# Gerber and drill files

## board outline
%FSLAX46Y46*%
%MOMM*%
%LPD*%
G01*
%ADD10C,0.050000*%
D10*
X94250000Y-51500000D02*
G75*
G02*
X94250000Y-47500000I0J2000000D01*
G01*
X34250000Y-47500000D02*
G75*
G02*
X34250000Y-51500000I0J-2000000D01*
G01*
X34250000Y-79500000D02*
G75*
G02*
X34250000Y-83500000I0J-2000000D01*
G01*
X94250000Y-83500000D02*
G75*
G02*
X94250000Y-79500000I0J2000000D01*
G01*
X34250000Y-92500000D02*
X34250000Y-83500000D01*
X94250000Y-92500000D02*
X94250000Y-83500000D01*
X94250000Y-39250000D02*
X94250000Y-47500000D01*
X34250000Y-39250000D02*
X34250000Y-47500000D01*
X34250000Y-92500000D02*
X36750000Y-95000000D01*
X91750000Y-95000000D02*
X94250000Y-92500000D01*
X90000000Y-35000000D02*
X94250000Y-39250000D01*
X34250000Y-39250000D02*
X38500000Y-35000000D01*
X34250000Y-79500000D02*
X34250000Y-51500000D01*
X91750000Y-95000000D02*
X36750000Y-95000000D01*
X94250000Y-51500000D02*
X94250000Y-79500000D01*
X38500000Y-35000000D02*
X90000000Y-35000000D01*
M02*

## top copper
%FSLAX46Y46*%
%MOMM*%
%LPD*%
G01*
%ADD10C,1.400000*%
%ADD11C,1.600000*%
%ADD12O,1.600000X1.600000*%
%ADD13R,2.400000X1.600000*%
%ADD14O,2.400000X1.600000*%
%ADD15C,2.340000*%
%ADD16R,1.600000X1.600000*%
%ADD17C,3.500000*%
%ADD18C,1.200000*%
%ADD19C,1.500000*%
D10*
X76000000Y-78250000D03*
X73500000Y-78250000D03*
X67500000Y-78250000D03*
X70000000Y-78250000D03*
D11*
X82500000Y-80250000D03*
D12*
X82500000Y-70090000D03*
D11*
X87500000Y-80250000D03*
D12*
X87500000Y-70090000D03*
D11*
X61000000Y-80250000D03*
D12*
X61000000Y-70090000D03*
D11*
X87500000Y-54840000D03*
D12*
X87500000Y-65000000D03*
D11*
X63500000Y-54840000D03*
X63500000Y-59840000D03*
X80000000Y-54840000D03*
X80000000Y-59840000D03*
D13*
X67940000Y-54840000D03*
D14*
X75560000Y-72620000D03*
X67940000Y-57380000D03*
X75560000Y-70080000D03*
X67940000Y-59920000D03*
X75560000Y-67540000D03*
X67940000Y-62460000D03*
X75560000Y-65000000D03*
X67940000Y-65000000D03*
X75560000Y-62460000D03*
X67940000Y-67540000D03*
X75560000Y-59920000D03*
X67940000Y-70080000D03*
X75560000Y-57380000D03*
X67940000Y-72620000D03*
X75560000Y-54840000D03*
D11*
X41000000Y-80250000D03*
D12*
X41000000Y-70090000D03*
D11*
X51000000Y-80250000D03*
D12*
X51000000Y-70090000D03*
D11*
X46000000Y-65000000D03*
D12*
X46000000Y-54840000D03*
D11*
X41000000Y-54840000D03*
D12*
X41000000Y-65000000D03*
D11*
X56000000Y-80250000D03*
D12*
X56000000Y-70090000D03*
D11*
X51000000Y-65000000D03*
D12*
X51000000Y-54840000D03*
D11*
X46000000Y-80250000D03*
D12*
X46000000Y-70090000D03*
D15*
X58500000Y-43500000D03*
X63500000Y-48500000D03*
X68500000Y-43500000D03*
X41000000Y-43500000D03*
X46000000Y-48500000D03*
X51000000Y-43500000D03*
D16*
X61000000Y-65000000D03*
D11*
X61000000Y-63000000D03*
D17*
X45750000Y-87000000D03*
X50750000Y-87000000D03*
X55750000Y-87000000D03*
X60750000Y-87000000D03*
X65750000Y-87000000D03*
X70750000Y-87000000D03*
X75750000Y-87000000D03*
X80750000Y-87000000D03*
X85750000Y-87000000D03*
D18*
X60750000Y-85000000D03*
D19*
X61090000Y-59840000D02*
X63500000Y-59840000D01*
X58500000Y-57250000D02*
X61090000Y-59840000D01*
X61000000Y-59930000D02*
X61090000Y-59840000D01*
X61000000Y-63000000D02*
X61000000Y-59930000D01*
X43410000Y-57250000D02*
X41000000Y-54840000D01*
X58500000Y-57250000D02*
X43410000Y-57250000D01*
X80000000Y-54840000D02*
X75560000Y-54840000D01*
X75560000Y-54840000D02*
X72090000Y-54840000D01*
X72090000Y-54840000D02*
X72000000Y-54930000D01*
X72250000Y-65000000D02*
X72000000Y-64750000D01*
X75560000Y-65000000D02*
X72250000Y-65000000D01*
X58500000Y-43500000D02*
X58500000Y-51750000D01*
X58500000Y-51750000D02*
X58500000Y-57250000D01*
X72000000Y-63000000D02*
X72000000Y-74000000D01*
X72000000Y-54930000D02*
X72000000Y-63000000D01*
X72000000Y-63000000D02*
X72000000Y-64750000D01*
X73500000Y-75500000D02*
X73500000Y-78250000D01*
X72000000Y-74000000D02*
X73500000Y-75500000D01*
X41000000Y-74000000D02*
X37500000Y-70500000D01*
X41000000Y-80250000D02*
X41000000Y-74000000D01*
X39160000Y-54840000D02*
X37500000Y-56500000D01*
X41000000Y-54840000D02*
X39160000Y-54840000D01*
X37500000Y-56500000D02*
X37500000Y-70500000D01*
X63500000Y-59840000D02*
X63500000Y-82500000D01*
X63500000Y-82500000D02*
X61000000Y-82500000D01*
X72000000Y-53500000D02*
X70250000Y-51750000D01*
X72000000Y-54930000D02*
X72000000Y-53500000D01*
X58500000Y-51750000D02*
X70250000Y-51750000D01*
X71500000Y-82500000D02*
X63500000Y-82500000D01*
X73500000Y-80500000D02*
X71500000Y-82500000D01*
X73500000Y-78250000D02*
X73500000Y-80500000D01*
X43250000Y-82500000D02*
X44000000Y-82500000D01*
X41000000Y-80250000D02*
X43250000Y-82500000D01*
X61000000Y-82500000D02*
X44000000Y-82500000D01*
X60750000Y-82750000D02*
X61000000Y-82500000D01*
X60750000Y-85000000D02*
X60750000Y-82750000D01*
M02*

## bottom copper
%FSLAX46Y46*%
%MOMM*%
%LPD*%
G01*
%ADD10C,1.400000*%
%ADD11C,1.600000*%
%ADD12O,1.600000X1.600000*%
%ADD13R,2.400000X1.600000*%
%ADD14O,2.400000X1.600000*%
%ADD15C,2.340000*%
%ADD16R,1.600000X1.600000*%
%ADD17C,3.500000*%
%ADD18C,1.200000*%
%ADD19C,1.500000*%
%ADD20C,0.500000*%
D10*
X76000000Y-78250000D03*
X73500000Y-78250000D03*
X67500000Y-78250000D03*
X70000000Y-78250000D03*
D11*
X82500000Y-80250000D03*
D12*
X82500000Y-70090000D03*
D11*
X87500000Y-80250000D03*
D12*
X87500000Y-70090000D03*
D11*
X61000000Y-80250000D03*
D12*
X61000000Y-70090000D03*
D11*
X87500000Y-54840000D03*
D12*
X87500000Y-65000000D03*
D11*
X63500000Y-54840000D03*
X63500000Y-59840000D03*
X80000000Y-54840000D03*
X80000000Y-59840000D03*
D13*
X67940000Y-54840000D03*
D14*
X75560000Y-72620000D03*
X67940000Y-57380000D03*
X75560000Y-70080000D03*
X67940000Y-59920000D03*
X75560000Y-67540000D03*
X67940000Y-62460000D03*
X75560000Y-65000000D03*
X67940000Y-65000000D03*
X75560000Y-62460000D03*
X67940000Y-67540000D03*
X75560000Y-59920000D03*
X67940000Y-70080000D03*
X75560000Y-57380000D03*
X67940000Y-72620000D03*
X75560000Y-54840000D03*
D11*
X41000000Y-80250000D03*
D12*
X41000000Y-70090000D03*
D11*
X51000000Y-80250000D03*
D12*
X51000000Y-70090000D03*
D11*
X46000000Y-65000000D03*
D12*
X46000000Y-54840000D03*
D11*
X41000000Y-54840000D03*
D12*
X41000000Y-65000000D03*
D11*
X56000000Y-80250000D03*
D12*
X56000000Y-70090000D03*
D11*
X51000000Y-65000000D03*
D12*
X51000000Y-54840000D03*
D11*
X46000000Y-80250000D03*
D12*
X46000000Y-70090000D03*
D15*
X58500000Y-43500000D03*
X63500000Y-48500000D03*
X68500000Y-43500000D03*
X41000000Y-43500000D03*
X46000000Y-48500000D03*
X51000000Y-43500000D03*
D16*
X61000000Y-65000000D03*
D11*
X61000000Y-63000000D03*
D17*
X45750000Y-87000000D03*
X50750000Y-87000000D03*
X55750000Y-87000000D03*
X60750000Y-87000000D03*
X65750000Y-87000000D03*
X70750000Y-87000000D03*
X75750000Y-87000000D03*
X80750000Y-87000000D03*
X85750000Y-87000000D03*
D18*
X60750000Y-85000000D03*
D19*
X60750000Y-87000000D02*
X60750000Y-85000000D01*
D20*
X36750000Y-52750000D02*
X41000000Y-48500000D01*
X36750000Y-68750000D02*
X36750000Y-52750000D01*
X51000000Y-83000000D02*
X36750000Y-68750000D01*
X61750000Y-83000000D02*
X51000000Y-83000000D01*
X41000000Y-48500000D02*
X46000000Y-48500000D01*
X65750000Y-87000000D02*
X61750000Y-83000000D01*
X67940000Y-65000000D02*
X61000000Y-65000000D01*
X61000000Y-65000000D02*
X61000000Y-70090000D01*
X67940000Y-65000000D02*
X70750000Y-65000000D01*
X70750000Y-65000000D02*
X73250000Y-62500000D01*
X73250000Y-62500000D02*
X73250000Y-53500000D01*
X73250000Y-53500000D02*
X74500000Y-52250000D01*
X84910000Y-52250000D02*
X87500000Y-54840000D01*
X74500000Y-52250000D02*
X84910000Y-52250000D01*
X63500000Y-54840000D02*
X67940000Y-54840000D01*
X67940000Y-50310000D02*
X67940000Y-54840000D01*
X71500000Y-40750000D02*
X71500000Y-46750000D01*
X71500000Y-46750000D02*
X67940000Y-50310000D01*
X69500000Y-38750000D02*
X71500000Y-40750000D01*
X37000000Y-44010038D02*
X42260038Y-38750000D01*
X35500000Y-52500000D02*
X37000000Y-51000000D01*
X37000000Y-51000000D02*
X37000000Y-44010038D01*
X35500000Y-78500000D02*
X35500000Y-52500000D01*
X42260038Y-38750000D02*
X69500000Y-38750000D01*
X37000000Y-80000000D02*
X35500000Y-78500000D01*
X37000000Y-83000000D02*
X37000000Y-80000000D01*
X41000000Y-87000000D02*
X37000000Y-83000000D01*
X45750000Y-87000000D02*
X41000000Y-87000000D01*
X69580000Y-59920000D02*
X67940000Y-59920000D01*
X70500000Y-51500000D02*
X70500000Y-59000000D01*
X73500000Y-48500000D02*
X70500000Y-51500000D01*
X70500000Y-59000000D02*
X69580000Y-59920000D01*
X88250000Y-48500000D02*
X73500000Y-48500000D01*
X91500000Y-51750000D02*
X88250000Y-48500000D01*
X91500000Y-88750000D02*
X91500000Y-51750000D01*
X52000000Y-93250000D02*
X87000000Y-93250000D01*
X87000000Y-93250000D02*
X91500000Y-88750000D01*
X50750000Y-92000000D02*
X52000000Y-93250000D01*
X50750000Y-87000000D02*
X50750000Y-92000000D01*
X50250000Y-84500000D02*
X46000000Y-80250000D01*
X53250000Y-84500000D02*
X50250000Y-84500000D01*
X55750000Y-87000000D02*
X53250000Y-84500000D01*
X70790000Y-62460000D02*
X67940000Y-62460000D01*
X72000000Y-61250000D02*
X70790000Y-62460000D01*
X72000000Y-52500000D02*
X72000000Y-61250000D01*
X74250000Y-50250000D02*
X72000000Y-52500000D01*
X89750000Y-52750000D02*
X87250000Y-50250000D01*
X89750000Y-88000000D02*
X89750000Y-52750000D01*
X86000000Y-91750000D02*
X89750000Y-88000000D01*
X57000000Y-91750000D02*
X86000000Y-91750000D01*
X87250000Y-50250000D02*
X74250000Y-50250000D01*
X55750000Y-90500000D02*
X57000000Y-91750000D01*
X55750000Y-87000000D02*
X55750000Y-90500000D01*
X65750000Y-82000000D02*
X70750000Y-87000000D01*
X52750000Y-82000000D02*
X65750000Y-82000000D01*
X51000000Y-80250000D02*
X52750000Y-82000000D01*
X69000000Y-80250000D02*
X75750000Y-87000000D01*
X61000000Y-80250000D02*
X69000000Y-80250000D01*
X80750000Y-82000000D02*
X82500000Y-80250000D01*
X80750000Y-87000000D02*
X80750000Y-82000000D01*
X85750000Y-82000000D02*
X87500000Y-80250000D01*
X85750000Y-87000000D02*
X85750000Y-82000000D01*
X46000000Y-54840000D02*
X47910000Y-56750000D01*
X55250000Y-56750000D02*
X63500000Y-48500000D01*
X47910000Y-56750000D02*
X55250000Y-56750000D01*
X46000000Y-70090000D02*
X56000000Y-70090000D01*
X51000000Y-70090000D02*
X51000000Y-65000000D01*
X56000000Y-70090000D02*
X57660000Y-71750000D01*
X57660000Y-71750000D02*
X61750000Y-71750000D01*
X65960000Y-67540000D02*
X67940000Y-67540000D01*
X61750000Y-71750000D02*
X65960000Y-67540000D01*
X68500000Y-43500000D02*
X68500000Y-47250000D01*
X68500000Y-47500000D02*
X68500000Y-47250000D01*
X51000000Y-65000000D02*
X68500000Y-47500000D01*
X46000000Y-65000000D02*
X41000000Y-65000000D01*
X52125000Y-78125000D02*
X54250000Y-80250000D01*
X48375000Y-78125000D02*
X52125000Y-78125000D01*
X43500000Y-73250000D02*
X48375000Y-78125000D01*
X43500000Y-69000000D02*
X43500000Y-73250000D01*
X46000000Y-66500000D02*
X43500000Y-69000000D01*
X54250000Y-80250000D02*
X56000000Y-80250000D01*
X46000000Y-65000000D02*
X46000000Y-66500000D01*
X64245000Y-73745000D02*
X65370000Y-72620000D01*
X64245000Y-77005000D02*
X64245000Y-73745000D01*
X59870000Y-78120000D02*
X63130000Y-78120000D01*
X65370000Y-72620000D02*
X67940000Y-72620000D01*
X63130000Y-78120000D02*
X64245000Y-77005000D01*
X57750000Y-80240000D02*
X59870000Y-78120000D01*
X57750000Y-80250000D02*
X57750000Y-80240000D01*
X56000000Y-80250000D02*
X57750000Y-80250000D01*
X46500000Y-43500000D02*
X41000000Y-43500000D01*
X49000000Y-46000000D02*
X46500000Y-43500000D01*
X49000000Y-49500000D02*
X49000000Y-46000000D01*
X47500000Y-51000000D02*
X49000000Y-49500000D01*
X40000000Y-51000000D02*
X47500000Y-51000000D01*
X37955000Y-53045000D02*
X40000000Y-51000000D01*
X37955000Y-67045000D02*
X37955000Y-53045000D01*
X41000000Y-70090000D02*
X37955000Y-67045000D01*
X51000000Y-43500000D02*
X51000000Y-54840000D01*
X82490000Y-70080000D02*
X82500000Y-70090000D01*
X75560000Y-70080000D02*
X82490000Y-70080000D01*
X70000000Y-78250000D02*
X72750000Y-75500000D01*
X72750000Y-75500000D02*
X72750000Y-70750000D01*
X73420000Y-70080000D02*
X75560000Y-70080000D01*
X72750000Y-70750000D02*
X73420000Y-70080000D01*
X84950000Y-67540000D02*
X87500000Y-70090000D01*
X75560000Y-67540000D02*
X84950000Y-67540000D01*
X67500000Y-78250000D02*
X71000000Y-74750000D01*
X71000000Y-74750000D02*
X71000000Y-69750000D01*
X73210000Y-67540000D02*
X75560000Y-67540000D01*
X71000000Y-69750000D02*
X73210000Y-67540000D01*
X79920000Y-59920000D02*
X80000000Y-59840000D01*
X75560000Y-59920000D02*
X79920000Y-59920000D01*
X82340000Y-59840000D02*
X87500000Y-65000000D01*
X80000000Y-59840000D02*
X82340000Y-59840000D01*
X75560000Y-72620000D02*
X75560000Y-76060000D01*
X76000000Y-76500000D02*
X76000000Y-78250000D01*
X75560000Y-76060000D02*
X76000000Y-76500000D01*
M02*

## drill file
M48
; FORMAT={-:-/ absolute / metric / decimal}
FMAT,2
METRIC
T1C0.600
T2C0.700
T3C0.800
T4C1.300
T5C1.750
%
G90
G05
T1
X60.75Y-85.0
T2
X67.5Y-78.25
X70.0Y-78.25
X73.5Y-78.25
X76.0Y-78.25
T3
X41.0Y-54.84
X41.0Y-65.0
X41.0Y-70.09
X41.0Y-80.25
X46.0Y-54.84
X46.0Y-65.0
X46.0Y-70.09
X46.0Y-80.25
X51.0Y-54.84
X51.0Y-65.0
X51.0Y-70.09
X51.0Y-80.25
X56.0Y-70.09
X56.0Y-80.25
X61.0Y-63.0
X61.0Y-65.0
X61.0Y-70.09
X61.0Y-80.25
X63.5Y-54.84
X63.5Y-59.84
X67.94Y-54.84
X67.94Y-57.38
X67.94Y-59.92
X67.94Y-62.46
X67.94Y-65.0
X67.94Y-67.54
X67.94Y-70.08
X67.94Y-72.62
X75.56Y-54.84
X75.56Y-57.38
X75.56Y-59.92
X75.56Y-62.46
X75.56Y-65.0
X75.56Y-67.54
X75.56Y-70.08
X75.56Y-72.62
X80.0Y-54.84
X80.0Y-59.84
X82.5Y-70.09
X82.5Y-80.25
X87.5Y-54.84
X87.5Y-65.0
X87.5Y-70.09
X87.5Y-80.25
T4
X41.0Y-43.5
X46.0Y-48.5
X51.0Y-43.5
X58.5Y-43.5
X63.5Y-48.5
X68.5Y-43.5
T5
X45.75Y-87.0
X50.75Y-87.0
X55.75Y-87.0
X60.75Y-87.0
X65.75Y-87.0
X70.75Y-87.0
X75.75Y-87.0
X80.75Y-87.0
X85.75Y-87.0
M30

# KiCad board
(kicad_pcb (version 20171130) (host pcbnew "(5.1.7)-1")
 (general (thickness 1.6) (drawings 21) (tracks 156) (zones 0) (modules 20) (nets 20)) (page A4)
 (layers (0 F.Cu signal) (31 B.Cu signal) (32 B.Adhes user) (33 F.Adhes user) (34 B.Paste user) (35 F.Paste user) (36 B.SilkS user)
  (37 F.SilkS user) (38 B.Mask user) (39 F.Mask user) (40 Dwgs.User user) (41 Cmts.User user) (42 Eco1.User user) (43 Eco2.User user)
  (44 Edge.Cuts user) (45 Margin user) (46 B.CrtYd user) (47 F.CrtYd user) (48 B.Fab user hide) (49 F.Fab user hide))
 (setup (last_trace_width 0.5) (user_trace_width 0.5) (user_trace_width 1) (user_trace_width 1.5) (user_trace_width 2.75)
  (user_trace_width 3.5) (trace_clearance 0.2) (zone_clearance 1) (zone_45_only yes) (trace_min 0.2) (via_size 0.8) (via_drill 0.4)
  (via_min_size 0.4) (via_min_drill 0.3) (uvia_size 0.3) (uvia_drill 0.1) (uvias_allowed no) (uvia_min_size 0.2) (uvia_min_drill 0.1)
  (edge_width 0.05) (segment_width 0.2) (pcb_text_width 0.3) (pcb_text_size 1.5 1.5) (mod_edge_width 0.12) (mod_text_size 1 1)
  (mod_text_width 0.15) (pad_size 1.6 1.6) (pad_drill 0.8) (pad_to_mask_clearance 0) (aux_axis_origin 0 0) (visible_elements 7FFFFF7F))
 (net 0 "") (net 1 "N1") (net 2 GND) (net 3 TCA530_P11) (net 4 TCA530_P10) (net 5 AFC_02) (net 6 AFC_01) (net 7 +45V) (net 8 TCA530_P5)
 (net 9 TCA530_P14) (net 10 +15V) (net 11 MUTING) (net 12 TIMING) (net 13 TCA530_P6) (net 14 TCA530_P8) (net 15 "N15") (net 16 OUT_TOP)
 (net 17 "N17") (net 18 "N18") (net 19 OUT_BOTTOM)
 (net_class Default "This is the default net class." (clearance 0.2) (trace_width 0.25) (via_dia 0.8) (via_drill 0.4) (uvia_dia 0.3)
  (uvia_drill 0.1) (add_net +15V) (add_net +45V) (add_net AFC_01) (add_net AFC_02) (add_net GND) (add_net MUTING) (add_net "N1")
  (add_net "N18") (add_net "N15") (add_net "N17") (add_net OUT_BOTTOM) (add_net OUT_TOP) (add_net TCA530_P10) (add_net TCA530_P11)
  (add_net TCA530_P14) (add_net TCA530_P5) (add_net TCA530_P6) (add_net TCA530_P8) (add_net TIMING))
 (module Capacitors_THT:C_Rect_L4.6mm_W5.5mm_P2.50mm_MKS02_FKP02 (layer F.Cu) (at 76 78.25 180)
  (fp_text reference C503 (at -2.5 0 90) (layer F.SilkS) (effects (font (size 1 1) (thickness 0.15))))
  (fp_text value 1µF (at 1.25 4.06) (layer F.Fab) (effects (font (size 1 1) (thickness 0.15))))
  (pad 1 thru_hole circle (at 0 0 180) (size 1.4 1.4) (drill 0.7) (layers *.Cu *.Mask) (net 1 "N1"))
  (pad 2 thru_hole circle (at 2.5 0 180) (size 1.4 1.4) (drill 0.7) (layers *.Cu *.Mask) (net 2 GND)))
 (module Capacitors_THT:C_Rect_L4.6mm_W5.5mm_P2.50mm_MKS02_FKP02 (layer F.Cu) (at 67.5 78.25)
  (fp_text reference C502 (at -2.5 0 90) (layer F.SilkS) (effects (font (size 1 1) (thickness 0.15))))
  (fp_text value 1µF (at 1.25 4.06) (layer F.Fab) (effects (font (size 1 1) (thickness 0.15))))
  (pad 1 thru_hole circle (at 0 0) (size 1.4 1.4) (drill 0.7) (layers *.Cu *.Mask) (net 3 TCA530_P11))
  (pad 2 thru_hole circle (at 2.5 0) (size 1.4 1.4) (drill 0.7) (layers *.Cu *.Mask) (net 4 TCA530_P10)))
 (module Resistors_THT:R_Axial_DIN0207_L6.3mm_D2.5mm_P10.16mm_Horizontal (layer F.Cu) (at 82.5 80.25 90)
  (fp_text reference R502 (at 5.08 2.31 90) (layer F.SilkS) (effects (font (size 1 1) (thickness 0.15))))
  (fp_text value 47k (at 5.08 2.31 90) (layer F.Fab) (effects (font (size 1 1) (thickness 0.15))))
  (pad 1 thru_hole circle (at 0 0 90) (size 1.6 1.6) (drill 0.8) (layers *.Cu *.Mask) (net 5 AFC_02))
  (pad 2 thru_hole oval (at 10.16 0 90) (size 1.6 1.6) (drill 0.8) (layers *.Cu *.Mask) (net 4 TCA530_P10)))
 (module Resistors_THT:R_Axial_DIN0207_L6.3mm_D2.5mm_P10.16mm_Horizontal (layer F.Cu) (at 87.5 80.25 90)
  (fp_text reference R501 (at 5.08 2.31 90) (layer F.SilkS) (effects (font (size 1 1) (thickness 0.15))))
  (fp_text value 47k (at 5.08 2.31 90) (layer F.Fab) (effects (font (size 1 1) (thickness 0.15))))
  (pad 1 thru_hole circle (at 0 0 90) (size 1.6 1.6) (drill 0.8) (layers *.Cu *.Mask) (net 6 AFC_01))
  (pad 2 thru_hole oval (at 10.16 0 90) (size 1.6 1.6) (drill 0.8) (layers *.Cu *.Mask) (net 3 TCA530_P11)))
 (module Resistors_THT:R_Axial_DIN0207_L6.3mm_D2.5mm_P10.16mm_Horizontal (layer F.Cu) (at 61 80.25 90)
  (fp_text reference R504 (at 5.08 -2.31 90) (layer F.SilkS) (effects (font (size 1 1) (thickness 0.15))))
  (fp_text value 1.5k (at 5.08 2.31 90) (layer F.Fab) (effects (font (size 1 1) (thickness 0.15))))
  (pad 1 thru_hole circle (at 0 0 90) (size 1.6 1.6) (drill 0.8) (layers *.Cu *.Mask) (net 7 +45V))
  (pad 2 thru_hole oval (at 10.16 0 90) (size 1.6 1.6) (drill 0.8) (layers *.Cu *.Mask) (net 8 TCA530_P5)))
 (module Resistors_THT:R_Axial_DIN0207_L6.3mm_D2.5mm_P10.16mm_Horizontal (layer F.Cu) (at 87.5 54.84 270)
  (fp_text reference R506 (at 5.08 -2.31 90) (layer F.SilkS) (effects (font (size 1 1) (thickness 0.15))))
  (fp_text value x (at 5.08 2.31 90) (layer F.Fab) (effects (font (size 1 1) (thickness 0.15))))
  (pad 1 thru_hole circle (at 0 0 270) (size 1.6 1.6) (drill 0.8) (layers *.Cu *.Mask) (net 8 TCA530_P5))
  (pad 2 thru_hole oval (at 10.16 0 270) (size 1.6 1.6) (drill 0.8) (layers *.Cu *.Mask) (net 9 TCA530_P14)))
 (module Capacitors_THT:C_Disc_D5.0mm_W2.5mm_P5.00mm (layer F.Cu) (at 63.5 54.84 270)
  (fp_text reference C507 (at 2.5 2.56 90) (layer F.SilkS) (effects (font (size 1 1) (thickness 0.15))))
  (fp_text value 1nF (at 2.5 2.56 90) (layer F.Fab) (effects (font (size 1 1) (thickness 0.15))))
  (pad 1 thru_hole circle (at 0 0 270) (size 1.6 1.6) (drill 0.8) (layers *.Cu *.Mask) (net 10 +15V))
  (pad 2 thru_hole circle (at 5 0 270) (size 1.6 1.6) (drill 0.8) (layers *.Cu *.Mask) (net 2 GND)))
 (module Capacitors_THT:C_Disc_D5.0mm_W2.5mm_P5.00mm (layer F.Cu) (at 80 54.84 270)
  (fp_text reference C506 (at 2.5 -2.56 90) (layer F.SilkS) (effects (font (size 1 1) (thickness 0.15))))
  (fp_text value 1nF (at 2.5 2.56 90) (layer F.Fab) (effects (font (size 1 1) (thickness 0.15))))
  (pad 1 thru_hole circle (at 0 0 270) (size 1.6 1.6) (drill 0.8) (layers *.Cu *.Mask) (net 2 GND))
  (pad 2 thru_hole circle (at 5 0 270) (size 1.6 1.6) (drill 0.8) (layers *.Cu *.Mask) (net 9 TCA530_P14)))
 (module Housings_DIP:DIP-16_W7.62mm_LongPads (layer F.Cu) (at 67.94 54.84)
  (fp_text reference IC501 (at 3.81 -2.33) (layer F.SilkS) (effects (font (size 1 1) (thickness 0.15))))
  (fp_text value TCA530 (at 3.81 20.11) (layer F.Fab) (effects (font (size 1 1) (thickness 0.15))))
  (pad 1 thru_hole rect (at 0 0) (size 2.4 1.6) (drill 0.8) (layers *.Cu *.Mask) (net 10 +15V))
  (pad 9 thru_hole oval (at 7.62 17.78) (size 2.4 1.6) (drill 0.8) (layers *.Cu *.Mask) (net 1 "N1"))
  (pad 2 thru_hole oval (at 0 2.54) (size 2.4 1.6) (drill 0.8) (layers *.Cu *.Mask))
  (pad 10 thru_hole oval (at 7.62 15.24) (size 2.4 1.6) (drill 0.8) (layers *.Cu *.Mask) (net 4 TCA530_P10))
  (pad 3 thru_hole oval (at 0 5.08) (size 2.4 1.6) (drill 0.8) (layers *.Cu *.Mask) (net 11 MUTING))
  (pad 11 thru_hole oval (at 7.62 12.7) (size 2.4 1.6) (drill 0.8) (layers *.Cu *.Mask) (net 3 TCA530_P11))
  (pad 4 thru_hole oval (at 0 7.62) (size 2.4 1.6) (drill 0.8) (layers *.Cu *.Mask) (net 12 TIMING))
  (pad 12 thru_hole oval (at 7.62 10.16) (size 2.4 1.6) (drill 0.8) (layers *.Cu *.Mask) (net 2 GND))
  (pad 5 thru_hole oval (at 0 10.16) (size 2.4 1.6) (drill 0.8) (layers *.Cu *.Mask) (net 8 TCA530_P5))
  (pad 13 thru_hole oval (at 7.62 7.62) (size 2.4 1.6) (drill 0.8) (layers *.Cu *.Mask))
  (pad 6 thru_hole oval (at 0 12.7) (size 2.4 1.6) (drill 0.8) (layers *.Cu *.Mask) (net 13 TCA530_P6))
  (pad 14 thru_hole oval (at 7.62 5.08) (size 2.4 1.6) (drill 0.8) (layers *.Cu *.Mask) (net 9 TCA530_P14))
  (pad 7 thru_hole oval (at 0 15.24) (size 2.4 1.6) (drill 0.8) (layers *.Cu *.Mask))
  (pad 15 thru_hole oval (at 7.62 2.54) (size 2.4 1.6) (drill 0.8) (layers *.Cu *.Mask))
  (pad 8 thru_hole oval (at 0 17.78) (size 2.4 1.6) (drill 0.8) (layers *.Cu *.Mask) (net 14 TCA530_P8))
  (pad 16 thru_hole oval (at 7.62 0) (size 2.4 1.6) (drill 0.8) (layers *.Cu *.Mask) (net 2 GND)))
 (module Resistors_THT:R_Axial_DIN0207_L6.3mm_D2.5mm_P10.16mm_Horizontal (layer F.Cu) (at 41 80.25 90)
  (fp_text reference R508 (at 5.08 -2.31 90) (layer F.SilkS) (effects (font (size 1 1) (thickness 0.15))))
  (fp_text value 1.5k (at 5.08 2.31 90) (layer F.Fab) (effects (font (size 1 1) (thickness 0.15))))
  (pad 1 thru_hole circle (at 0 0 90) (size 1.6 1.6) (drill 0.8) (layers *.Cu *.Mask) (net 2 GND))
  (pad 2 thru_hole oval (at 10.16 0 90) (size 1.6 1.6) (drill 0.8) (layers *.Cu *.Mask) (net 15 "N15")))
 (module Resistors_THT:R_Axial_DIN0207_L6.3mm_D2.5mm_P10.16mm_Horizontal (layer F.Cu) (at 51 80.25 90)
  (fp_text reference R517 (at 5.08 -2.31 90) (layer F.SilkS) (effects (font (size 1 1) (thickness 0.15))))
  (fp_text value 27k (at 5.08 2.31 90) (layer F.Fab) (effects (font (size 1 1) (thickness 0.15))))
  (pad 1 thru_hole circle (at 0 0 90) (size 1.6 1.6) (drill 0.8) (layers *.Cu *.Mask) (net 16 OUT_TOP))
  (pad 2 thru_hole oval (at 10.16 0 90) (size 1.6 1.6) (drill 0.8) (layers *.Cu *.Mask) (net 13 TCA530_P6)))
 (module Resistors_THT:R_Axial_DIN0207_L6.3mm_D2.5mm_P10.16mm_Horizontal (layer F.Cu) (at 46 65 90)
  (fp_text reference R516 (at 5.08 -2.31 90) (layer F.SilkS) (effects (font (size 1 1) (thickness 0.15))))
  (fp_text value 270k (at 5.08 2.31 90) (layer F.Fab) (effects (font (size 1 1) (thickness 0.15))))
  (pad 1 thru_hole circle (at 0 0 90) (size 1.6 1.6) (drill 0.8) (layers *.Cu *.Mask) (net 14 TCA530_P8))
  (pad 2 thru_hole oval (at 10.16 0 90) (size 1.6 1.6) (drill 0.8) (layers *.Cu *.Mask) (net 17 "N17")))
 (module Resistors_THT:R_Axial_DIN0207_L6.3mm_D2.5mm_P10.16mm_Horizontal (layer F.Cu) (at 41 54.84 270)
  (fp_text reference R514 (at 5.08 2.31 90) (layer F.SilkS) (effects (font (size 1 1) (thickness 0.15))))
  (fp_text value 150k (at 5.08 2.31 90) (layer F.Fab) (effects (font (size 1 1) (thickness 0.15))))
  (pad 1 thru_hole circle (at 0 0 270) (size 1.6 1.6) (drill 0.8) (layers *.Cu *.Mask) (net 2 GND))
  (pad 2 thru_hole oval (at 10.16 0 270) (size 1.6 1.6) (drill 0.8) (layers *.Cu *.Mask) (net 14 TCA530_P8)))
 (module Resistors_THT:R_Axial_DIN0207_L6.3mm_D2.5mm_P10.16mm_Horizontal (layer F.Cu) (at 56 80.25 90)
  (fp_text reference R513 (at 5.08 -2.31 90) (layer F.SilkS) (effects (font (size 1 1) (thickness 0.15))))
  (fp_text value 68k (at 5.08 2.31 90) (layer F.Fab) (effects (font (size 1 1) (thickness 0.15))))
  (pad 1 thru_hole circle (at 0 0 90) (size 1.6 1.6) (drill 0.8) (layers *.Cu *.Mask) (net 14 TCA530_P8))
  (pad 2 thru_hole oval (at 10.16 0 90) (size 1.6 1.6) (drill 0.8) (layers *.Cu *.Mask) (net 13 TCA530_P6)))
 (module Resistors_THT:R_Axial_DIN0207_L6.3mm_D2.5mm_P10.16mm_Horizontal (layer F.Cu) (at 51 65 90)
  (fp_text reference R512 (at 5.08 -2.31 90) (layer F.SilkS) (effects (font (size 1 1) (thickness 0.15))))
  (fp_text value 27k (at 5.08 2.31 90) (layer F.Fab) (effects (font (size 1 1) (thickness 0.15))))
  (pad 1 thru_hole circle (at 0 0 90) (size 1.6 1.6) (drill 0.8) (layers *.Cu *.Mask) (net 13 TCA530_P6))
  (pad 2 thru_hole oval (at 10.16 0 90) (size 1.6 1.6) (drill 0.8) (layers *.Cu *.Mask) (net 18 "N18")))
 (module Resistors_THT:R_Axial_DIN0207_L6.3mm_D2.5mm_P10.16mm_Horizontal (layer F.Cu) (at 46 80.25 90)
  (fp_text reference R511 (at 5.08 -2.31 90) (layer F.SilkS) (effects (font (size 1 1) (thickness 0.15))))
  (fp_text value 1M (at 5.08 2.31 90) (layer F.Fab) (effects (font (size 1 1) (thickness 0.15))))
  (pad 1 thru_hole circle (at 0 0 90) (size 1.6 1.6) (drill 0.8) (layers *.Cu *.Mask) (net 12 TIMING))
  (pad 2 thru_hole oval (at 10.16 0 90) (size 1.6 1.6) (drill 0.8) (layers *.Cu *.Mask) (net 13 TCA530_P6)))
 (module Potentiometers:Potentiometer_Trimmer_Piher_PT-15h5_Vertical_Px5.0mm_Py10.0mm (layer F.Cu) (at 68.5 43.5 270)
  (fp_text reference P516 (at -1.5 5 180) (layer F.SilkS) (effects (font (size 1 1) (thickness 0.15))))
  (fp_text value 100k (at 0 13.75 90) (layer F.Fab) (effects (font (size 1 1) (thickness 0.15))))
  (pad 3 thru_hole circle (at 0 10 270) (size 2.34 2.34) (drill 1.3) (layers *.Cu *.Mask) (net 2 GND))
  (pad 2 thru_hole circle (at 5 5 270) (size 2.34 2.34) (drill 1.3) (layers *.Cu *.Mask) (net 17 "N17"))
  (pad 1 thru_hole circle (at 0 0 270) (size 2.34 2.34) (drill 1.3) (layers *.Cu *.Mask) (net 13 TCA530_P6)))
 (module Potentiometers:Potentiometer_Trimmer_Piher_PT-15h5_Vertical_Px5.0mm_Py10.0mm (layer F.Cu) (at 51 43.5 270)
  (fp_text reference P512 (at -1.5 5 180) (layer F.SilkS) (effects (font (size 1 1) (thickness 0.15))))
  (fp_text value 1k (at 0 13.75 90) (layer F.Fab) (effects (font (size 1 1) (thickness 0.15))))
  (pad 3 thru_hole circle (at 0 10 270) (size 2.34 2.34) (drill 1.3) (layers *.Cu *.Mask) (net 15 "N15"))
  (pad 2 thru_hole circle (at 5 5 270) (size 2.34 2.34) (drill 1.3) (layers *.Cu *.Mask) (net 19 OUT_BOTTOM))
  (pad 1 thru_hole circle (at 0 0 270) (size 2.34 2.34) (drill 1.3) (layers *.Cu *.Mask) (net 18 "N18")))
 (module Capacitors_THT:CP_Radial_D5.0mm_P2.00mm (layer F.Cu) (at 61 65 90)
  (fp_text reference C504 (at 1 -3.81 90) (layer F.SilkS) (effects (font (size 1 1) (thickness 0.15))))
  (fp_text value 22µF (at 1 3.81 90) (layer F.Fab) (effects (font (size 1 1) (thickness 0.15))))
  (pad 1 thru_hole rect (at 0 0 90) (size 1.6 1.6) (drill 0.8) (layers *.Cu *.Mask) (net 8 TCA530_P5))
  (pad 2 thru_hole circle (at 2 0 90) (size 1.6 1.6) (drill 0.8) (layers *.Cu *.Mask) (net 2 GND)))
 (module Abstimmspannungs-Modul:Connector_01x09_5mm (layer F.Cu) (at 85.75 87)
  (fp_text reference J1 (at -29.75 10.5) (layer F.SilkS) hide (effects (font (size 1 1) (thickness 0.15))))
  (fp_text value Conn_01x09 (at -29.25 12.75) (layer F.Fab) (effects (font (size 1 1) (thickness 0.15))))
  (pad 9 thru_hole circle (at -40 0 180) (size 3.5 3.5) (drill 1.75) (layers B.Cu B.Mask) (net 10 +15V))
  (pad 8 thru_hole circle (at -35 0 180) (size 3.5 3.5) (drill 1.75) (layers B.Cu B.Mask) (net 11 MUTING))
  (pad 7 thru_hole circle (at -30 0 180) (size 3.5 3.5) (drill 1.75) (layers B.Cu B.Mask) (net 12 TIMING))
  (pad 6 thru_hole circle (at -25 0 180) (size 3.5 3.5) (drill 1.75) (layers B.Cu B.Mask) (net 2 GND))
  (pad 5 thru_hole circle (at -20 0 180) (size 3.5 3.5) (drill 1.75) (layers B.Cu B.Mask) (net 19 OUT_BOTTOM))
  (pad 4 thru_hole circle (at -15 0 180) (size 3.5 3.5) (drill 1.75) (layers B.Cu B.Mask) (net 16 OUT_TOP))
  (pad 3 thru_hole circle (at -10 0 180) (size 3.5 3.5) (drill 1.75) (layers B.Cu B.Mask) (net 7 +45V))
  (pad 2 thru_hole circle (at -5 0 180) (size 3.5 3.5) (drill 1.75) (layers B.Cu B.Mask) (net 5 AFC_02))
  (pad 1 thru_hole circle (at 0 0 180) (size 3.5 3.5) (drill 1.75) (layers B.Cu B.Mask) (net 6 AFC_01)))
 (gr_arc (start 94.25 49.5) (end 94.25 47.5) (angle -180) (layer Edge.Cuts) (width 0.05))
 (gr_arc (start 34.25 49.5) (end 34.25 51.5) (angle -180) (layer Edge.Cuts) (width 0.05))
 (gr_arc (start 34.25 81.5) (end 34.25 83.5) (angle -180) (layer Edge.Cuts) (width 0.05))
 (gr_arc (start 94.25 81.5) (end 94.25 79.5) (angle -180) (layer Edge.Cuts) (width 0.05))
 (gr_line (start 34.25 92.5) (end 34.25 83.5) (layer Edge.Cuts) (width 0.05))
 (gr_line (start 94.25 92.5) (end 94.25 83.5) (layer Edge.Cuts) (width 0.05))
 (gr_line (start 94.25 39.25) (end 94.25 47.5) (layer Edge.Cuts) (width 0.05))
 (gr_line (start 34.25 39.25) (end 34.25 47.5) (layer Edge.Cuts) (width 0.05))
 (gr_line (start 34.25 92.5) (end 36.75 95) (layer Edge.Cuts) (width 0.05))
 (gr_line (start 91.75 95) (end 94.25 92.5) (layer Edge.Cuts) (width 0.05))
 (gr_line (start 90 35) (end 94.25 39.25) (layer Edge.Cuts) (width 0.05))
 (gr_line (start 34.25 39.25) (end 38.5 35) (layer Edge.Cuts) (width 0.05))
 (gr_line (start 34.25 79.5) (end 34.25 51.5) (layer Edge.Cuts) (width 0.05))
 (gr_line (start 91.75 95) (end 36.75 95) (layer Edge.Cuts) (width 0.05))
 (gr_line (start 94.25 51.5) (end 94.25 79.5) (layer Edge.Cuts) (width 0.05))
 (gr_line (start 38.5 35) (end 90 35) (layer Edge.Cuts) (width 0.05))
 (segment (start 61.09 59.84) (end 63.5 59.84) (width 1.5) (layer F.Cu) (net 2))
 (segment (start 58.5 57.25) (end 61.09 59.84) (width 1.5) (layer F.Cu) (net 2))
 (segment (start 61 59.93) (end 61.09 59.84) (width 1.5) (layer F.Cu) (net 2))
 (segment (start 61 63) (end 61 59.93) (width 1.5) (layer F.Cu) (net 2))
 (segment (start 43.41 57.25) (end 41 54.84) (width 1.5) (layer F.Cu) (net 2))
 (segment (start 58.5 57.25) (end 43.41 57.25) (width 1.5) (layer F.Cu) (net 2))
 (segment (start 80 54.84) (end 75.56 54.84) (width 1.5) (layer F.Cu) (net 2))
 (segment (start 75.56 54.84) (end 72.09 54.84) (width 1.5) (layer F.Cu) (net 2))
 (segment (start 72.09 54.84) (end 72 54.93) (width 1.5) (layer F.Cu) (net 2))
 (segment (start 72.25 65) (end 72 64.75) (width 1.5) (layer F.Cu) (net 2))
 (segment (start 75.56 65) (end 72.25 65) (width 1.5) (layer F.Cu) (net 2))
 (segment (start 58.5 43.5) (end 58.5 51.75) (width 1.5) (layer F.Cu) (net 2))
 (segment (start 58.5 51.75) (end 58.5 57.25) (width 1.5) (layer F.Cu) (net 2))
 (segment (start 72 63) (end 72 74) (width 1.5) (layer F.Cu) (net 2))
 (segment (start 72 54.93) (end 72 63) (width 1.5) (layer F.Cu) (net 2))
 (segment (start 72 63) (end 72 64.75) (width 1.5) (layer F.Cu) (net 2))
 (segment (start 73.5 75.5) (end 73.5 78.25) (width 1.5) (layer F.Cu) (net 2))
 (segment (start 72 74) (end 73.5 75.5) (width 1.5) (layer F.Cu) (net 2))
 (segment (start 41 74) (end 37.5 70.5) (width 1.5) (layer F.Cu) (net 2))
 (segment (start 41 80.25) (end 41 74) (width 1.5) (layer F.Cu) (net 2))
 (segment (start 39.16 54.84) (end 37.5 56.5) (width 1.5) (layer F.Cu) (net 2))
 (segment (start 41 54.84) (end 39.16 54.84) (width 1.5) (layer F.Cu) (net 2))
 (segment (start 37.5 56.5) (end 37.5 70.5) (width 1.5) (layer F.Cu) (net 2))
 (segment (start 63.5 59.84) (end 63.5 82.5) (width 1.5) (layer F.Cu) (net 2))
 (segment (start 63.5 82.5) (end 61 82.5) (width 1.5) (layer F.Cu) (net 2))
 (segment (start 72 53.5) (end 70.25 51.75) (width 1.5) (layer F.Cu) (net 2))
 (segment (start 72 54.93) (end 72 53.5) (width 1.5) (layer F.Cu) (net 2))
 (segment (start 58.5 51.75) (end 70.25 51.75) (width 1.5) (layer F.Cu) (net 2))
 (segment (start 71.5 82.5) (end 63.5 82.5) (width 1.5) (layer F.Cu) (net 2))
 (segment (start 73.5 80.5) (end 71.5 82.5) (width 1.5) (layer F.Cu) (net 2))
 (segment (start 73.5 78.25) (end 73.5 80.5) (width 1.5) (layer F.Cu) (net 2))
 (segment (start 43.25 82.5) (end 44 82.5) (width 1.5) (layer F.Cu) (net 2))
 (segment (start 41 80.25) (end 43.25 82.5) (width 1.5) (layer F.Cu) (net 2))
 (segment (start 61 82.5) (end 44 82.5) (width 1.5) (layer F.Cu) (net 2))
 (segment (start 60.75 87) (end 60.75 85) (width 1.5) (layer B.Cu) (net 2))
 (via (at 60.75 85) (size 1.2) (drill 0.6) (layers F.Cu B.Cu) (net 2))
 (segment (start 60.75 82.75) (end 61 82.5) (width 1.5) (layer F.Cu) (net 2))
 (segment (start 60.75 85) (end 60.75 82.75) (width 1.5) (layer F.Cu) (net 2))
 (segment (start 36.75 52.75) (end 41 48.5) (width 0.5) (layer B.Cu) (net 19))
 (segment (start 36.75 68.75) (end 36.75 52.75) (width 0.5) (layer B.Cu) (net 19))
 (segment (start 51 83) (end 36.75 68.75) (width 0.5) (layer B.Cu) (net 19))
 (segment (start 61.75 83) (end 51 83) (width 0.5) (layer B.Cu) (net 19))
 (segment (start 41 48.5) (end 46 48.5) (width 0.5) (layer B.Cu) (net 19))
 (segment (start 65.75 87) (end 61.75 83) (width 0.5) (layer B.Cu) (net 19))
 (segment (start 67.94 65) (end 61 65) (width 0.5) (layer B.Cu) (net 8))
 (segment (start 61 65) (end 61 70.09) (width 0.5) (layer B.Cu) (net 8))
 (segment (start 67.94 65) (end 70.75 65) (width 0.5) (layer B.Cu) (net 8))
 (segment (start 70.75 65) (end 73.25 62.5) (width 0.5) (layer B.Cu) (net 8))
 (segment (start 73.25 62.5) (end 73.25 53.5) (width 0.5) (layer B.Cu) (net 8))
 (segment (start 73.25 53.5) (end 74.5 52.25) (width 0.5) (layer B.Cu) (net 8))
 (segment (start 84.91 52.25) (end 87.5 54.84) (width 0.5) (layer B.Cu) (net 8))
 (segment (start 74.5 52.25) (end 84.91 52.25) (width 0.5) (layer B.Cu) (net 8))
 (segment (start 63.5 54.84) (end 67.94 54.84) (width 0.5) (layer B.Cu) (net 10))
 (segment (start 67.94 50.31) (end 67.94 54.84) (width 0.5) (layer B.Cu) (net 10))
 (segment (start 71.5 40.75) (end 71.5 46.75) (width 0.5) (layer B.Cu) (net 10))
 (segment (start 71.5 46.75) (end 67.94 50.31) (width 0.5) (layer B.Cu) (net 10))
 (segment (start 69.5 38.75) (end 71.5 40.75) (width 0.5) (layer B.Cu) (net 10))
 (segment (start 37 44.010038) (end 42.260038 38.75) (width 0.5) (layer B.Cu) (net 10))
 (segment (start 35.5 52.5) (end 37 51) (width 0.5) (layer B.Cu) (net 10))
 (segment (start 37 51) (end 37 44.010038) (width 0.5) (layer B.Cu) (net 10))
 (segment (start 35.5 78.5) (end 35.5 52.5) (width 0.5) (layer B.Cu) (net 10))
 (segment (start 42.260038 38.75) (end 69.5 38.75) (width 0.5) (layer B.Cu) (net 10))
 (segment (start 37 80) (end 35.5 78.5) (width 0.5) (layer B.Cu) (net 10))
 (segment (start 37 83) (end 37 80) (width 0.5) (layer B.Cu) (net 10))
 (segment (start 41 87) (end 37 83) (width 0.5) (layer B.Cu) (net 10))
 (segment (start 45.75 87) (end 41 87) (width 0.5) (layer B.Cu) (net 10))
 (segment (start 69.58 59.92) (end 67.94 59.92) (width 0.5) (layer B.Cu) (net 11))
 (segment (start 70.5 51.5) (end 70.5 59) (width 0.5) (layer B.Cu) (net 11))
 (segment (start 73.5 48.5) (end 70.5 51.5) (width 0.5) (layer B.Cu) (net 11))
 (segment (start 70.5 59) (end 69.58 59.92) (width 0.5) (layer B.Cu) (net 11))
 (segment (start 88.25 48.5) (end 73.5 48.5) (width 0.5) (layer B.Cu) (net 11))
 (segment (start 91.5 51.75) (end 88.25 48.5) (width 0.5) (layer B.Cu) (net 11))
 (segment (start 91.5 88.75) (end 91.5 51.75) (width 0.5) (layer B.Cu) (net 11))
 (segment (start 52 93.25) (end 87 93.25) (width 0.5) (layer B.Cu) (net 11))
 (segment (start 87 93.25) (end 91.5 88.75) (width 0.5) (layer B.Cu) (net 11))
 (segment (start 50.75 92) (end 52 93.25) (width 0.5) (layer B.Cu) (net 11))
 (segment (start 50.75 87) (end 50.75 92) (width 0.5) (layer B.Cu) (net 11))
 (segment (start 50.25 84.5) (end 46 80.25) (width 0.5) (layer B.Cu) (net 12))
 (segment (start 53.25 84.5) (end 50.25 84.5) (width 0.5) (layer B.Cu) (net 12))
 (segment (start 55.75 87) (end 53.25 84.5) (width 0.5) (layer B.Cu) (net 12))
 (segment (start 70.79 62.46) (end 67.94 62.46) (width 0.5) (layer B.Cu) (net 12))
 (segment (start 72 61.25) (end 70.79 62.46) (width 0.5) (layer B.Cu) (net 12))
 (segment (start 72 52.5) (end 72 61.25) (width 0.5) (layer B.Cu) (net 12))
 (segment (start 74.25 50.25) (end 72 52.5) (width 0.5) (layer B.Cu) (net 12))
 (segment (start 89.75 52.75) (end 87.25 50.25) (width 0.5) (layer B.Cu) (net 12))
 (segment (start 89.75 88) (end 89.75 52.75) (width 0.5) (layer B.Cu) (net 12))
 (segment (start 86 91.75) (end 89.75 88) (width 0.5) (layer B.Cu) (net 12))
 (segment (start 57 91.75) (end 86 91.75) (width 0.5) (layer B.Cu) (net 12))
 (segment (start 87.25 50.25) (end 74.25 50.25) (width 0.5) (layer B.Cu) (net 12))
 (segment (start 55.75 90.5) (end 57 91.75) (width 0.5) (layer B.Cu) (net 12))
 (segment (start 55.75 87) (end 55.75 90.5) (width 0.5) (layer B.Cu) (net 12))
 (segment (start 65.75 82) (end 70.75 87) (width 0.5) (layer B.Cu) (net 16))
 (segment (start 52.75 82) (end 65.75 82) (width 0.5) (layer B.Cu) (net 16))
 (segment (start 51 80.25) (end 52.75 82) (width 0.5) (layer B.Cu) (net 16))
 (segment (start 69 80.25) (end 75.75 87) (width 0.5) (layer B.Cu) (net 7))
 (segment (start 61 80.25) (end 69 80.25) (width 0.5) (layer B.Cu) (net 7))
 (segment (start 80.75 82) (end 82.5 80.25) (width 0.5) (layer B.Cu) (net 5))
 (segment (start 80.75 87) (end 80.75 82) (width 0.5) (layer B.Cu) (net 5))
 (segment (start 85.75 82) (end 87.5 80.25) (width 0.5) (layer B.Cu) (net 6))
 (segment (start 85.75 87) (end 85.75 82) (width 0.5) (layer B.Cu) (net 6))
 (segment (start 46 54.84) (end 47.91 56.75) (width 0.5) (layer B.Cu) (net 17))
 (segment (start 55.25 56.75) (end 63.5 48.5) (width 0.5) (layer B.Cu) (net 17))
 (segment (start 47.91 56.75) (end 55.25 56.75) (width 0.5) (layer B.Cu) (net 17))
 (segment (start 46 70.09) (end 56 70.09) (width 0.5) (layer B.Cu) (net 13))
 (segment (start 51 70.09) (end 51 65) (width 0.5) (layer B.Cu) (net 13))
 (segment (start 56 70.09) (end 57.66 71.75) (width 0.5) (layer B.Cu) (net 13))
 (segment (start 57.66 71.75) (end 61.75 71.75) (width 0.5) (layer B.Cu) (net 13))
 (segment (start 65.96 67.54) (end 67.94 67.54) (width 0.5) (layer B.Cu) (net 13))
 (segment (start 61.75 71.75) (end 65.96 67.54) (width 0.5) (layer B.Cu) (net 13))
 (segment (start 68.5 43.5) (end 68.5 47.25) (width 0.5) (layer B.Cu) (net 13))
 (segment (start 68.5 47.5) (end 68.5 47.25) (width 0.5) (layer B.Cu) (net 13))
 (segment (start 51 65) (end 68.5 47.5) (width 0.5) (layer B.Cu) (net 13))
 (segment (start 46 65) (end 41 65) (width 0.5) (layer B.Cu) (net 14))
 (segment (start 52.125 78.125) (end 54.25 80.25) (width 0.5) (layer B.Cu) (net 14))
 (segment (start 48.375 78.125) (end 52.125 78.125) (width 0.5) (layer B.Cu) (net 14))
 (segment (start 43.5 73.25) (end 48.375 78.125) (width 0.5) (layer B.Cu) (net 14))
 (segment (start 43.5 69) (end 43.5 73.25) (width 0.5) (layer B.Cu) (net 14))
 (segment (start 46 66.5) (end 43.5 69) (width 0.5) (layer B.Cu) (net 14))
 (segment (start 54.25 80.25) (end 56 80.25) (width 0.5) (layer B.Cu) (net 14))
 (segment (start 46 65) (end 46 66.5) (width 0.5) (layer B.Cu) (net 14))
 (segment (start 64.245 73.745) (end 65.37 72.62) (width 0.5) (layer B.Cu) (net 14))
 (segment (start 64.245 77.005) (end 64.245 73.745) (width 0.5) (layer B.Cu) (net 14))
 (segment (start 59.87 78.12) (end 63.13 78.12) (width 0.5) (layer B.Cu) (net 14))
 (segment (start 65.37 72.62) (end 67.94 72.62) (width 0.5) (layer B.Cu) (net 14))
 (segment (start 63.13 78.12) (end 64.245 77.005) (width 0.5) (layer B.Cu) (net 14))
 (segment (start 57.75 80.24) (end 59.87 78.12) (width 0.5) (layer B.Cu) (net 14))
 (segment (start 57.75 80.25) (end 57.75 80.24) (width 0.5) (layer B.Cu) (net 14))
 (segment (start 56 80.25) (end 57.75 80.25) (width 0.5) (layer B.Cu) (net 14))
 (segment (start 46.5 43.5) (end 41 43.5) (width 0.5) (layer B.Cu) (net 15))
 (segment (start 49 46) (end 46.5 43.5) (width 0.5) (layer B.Cu) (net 15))
 (segment (start 49 49.5) (end 49 46) (width 0.5) (layer B.Cu) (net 15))
 (segment (start 47.5 51) (end 49 49.5) (width 0.5) (layer B.Cu) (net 15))
 (segment (start 40 51) (end 47.5 51) (width 0.5) (layer B.Cu) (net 15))
 (segment (start 37.955 53.045) (end 40 51) (width 0.5) (layer B.Cu) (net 15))
 (segment (start 37.955 67.045) (end 37.955 53.045) (width 0.5) (layer B.Cu) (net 15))
 (segment (start 41 70.09) (end 37.955 67.045) (width 0.5) (layer B.Cu) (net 15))
 (segment (start 51 43.5) (end 51 54.84) (width 0.5) (layer B.Cu) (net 18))
 (segment (start 82.49 70.08) (end 82.5 70.09) (width 0.5) (layer B.Cu) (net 4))
 (segment (start 75.56 70.08) (end 82.49 70.08) (width 0.5) (layer B.Cu) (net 4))
 (segment (start 70 78.25) (end 72.75 75.5) (width 0.5) (layer B.Cu) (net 4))
 (segment (start 72.75 75.5) (end 72.75 70.75) (width 0.5) (layer B.Cu) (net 4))
 (segment (start 73.42 70.08) (end 75.56 70.08) (width 0.5) (layer B.Cu) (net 4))
 (segment (start 72.75 70.75) (end 73.42 70.08) (width 0.5) (layer B.Cu) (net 4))
 (segment (start 84.95 67.54) (end 87.5 70.09) (width 0.5) (layer B.Cu) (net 3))
 (segment (start 75.56 67.54) (end 84.95 67.54) (width 0.5) (layer B.Cu) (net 3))
 (segment (start 67.5 78.25) (end 71 74.75) (width 0.5) (layer B.Cu) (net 3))
 (segment (start 71 74.75) (end 71 69.75) (width 0.5) (layer B.Cu) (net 3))
 (segment (start 73.21 67.54) (end 75.56 67.54) (width 0.5) (layer B.Cu) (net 3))
 (segment (start 71 69.75) (end 73.21 67.54) (width 0.5) (layer B.Cu) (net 3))
 (segment (start 79.92 59.92) (end 80 59.84) (width 0.5) (layer B.Cu) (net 9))
 (segment (start 75.56 59.92) (end 79.92 59.92) (width 0.5) (layer B.Cu) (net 9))
 (segment (start 82.34 59.84) (end 87.5 65) (width 0.5) (layer B.Cu) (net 9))
 (segment (start 80 59.84) (end 82.34 59.84) (width 0.5) (layer B.Cu) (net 9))
 (segment (start 75.56 72.62) (end 75.56 76.06) (width 0.5) (layer B.Cu) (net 1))
 (segment (start 76 76.5) (end 76 78.25) (width 0.5) (layer B.Cu) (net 1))
 (segment (start 75.56 76.06) (end 76 76.5) (width 0.5) (layer B.Cu) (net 1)))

